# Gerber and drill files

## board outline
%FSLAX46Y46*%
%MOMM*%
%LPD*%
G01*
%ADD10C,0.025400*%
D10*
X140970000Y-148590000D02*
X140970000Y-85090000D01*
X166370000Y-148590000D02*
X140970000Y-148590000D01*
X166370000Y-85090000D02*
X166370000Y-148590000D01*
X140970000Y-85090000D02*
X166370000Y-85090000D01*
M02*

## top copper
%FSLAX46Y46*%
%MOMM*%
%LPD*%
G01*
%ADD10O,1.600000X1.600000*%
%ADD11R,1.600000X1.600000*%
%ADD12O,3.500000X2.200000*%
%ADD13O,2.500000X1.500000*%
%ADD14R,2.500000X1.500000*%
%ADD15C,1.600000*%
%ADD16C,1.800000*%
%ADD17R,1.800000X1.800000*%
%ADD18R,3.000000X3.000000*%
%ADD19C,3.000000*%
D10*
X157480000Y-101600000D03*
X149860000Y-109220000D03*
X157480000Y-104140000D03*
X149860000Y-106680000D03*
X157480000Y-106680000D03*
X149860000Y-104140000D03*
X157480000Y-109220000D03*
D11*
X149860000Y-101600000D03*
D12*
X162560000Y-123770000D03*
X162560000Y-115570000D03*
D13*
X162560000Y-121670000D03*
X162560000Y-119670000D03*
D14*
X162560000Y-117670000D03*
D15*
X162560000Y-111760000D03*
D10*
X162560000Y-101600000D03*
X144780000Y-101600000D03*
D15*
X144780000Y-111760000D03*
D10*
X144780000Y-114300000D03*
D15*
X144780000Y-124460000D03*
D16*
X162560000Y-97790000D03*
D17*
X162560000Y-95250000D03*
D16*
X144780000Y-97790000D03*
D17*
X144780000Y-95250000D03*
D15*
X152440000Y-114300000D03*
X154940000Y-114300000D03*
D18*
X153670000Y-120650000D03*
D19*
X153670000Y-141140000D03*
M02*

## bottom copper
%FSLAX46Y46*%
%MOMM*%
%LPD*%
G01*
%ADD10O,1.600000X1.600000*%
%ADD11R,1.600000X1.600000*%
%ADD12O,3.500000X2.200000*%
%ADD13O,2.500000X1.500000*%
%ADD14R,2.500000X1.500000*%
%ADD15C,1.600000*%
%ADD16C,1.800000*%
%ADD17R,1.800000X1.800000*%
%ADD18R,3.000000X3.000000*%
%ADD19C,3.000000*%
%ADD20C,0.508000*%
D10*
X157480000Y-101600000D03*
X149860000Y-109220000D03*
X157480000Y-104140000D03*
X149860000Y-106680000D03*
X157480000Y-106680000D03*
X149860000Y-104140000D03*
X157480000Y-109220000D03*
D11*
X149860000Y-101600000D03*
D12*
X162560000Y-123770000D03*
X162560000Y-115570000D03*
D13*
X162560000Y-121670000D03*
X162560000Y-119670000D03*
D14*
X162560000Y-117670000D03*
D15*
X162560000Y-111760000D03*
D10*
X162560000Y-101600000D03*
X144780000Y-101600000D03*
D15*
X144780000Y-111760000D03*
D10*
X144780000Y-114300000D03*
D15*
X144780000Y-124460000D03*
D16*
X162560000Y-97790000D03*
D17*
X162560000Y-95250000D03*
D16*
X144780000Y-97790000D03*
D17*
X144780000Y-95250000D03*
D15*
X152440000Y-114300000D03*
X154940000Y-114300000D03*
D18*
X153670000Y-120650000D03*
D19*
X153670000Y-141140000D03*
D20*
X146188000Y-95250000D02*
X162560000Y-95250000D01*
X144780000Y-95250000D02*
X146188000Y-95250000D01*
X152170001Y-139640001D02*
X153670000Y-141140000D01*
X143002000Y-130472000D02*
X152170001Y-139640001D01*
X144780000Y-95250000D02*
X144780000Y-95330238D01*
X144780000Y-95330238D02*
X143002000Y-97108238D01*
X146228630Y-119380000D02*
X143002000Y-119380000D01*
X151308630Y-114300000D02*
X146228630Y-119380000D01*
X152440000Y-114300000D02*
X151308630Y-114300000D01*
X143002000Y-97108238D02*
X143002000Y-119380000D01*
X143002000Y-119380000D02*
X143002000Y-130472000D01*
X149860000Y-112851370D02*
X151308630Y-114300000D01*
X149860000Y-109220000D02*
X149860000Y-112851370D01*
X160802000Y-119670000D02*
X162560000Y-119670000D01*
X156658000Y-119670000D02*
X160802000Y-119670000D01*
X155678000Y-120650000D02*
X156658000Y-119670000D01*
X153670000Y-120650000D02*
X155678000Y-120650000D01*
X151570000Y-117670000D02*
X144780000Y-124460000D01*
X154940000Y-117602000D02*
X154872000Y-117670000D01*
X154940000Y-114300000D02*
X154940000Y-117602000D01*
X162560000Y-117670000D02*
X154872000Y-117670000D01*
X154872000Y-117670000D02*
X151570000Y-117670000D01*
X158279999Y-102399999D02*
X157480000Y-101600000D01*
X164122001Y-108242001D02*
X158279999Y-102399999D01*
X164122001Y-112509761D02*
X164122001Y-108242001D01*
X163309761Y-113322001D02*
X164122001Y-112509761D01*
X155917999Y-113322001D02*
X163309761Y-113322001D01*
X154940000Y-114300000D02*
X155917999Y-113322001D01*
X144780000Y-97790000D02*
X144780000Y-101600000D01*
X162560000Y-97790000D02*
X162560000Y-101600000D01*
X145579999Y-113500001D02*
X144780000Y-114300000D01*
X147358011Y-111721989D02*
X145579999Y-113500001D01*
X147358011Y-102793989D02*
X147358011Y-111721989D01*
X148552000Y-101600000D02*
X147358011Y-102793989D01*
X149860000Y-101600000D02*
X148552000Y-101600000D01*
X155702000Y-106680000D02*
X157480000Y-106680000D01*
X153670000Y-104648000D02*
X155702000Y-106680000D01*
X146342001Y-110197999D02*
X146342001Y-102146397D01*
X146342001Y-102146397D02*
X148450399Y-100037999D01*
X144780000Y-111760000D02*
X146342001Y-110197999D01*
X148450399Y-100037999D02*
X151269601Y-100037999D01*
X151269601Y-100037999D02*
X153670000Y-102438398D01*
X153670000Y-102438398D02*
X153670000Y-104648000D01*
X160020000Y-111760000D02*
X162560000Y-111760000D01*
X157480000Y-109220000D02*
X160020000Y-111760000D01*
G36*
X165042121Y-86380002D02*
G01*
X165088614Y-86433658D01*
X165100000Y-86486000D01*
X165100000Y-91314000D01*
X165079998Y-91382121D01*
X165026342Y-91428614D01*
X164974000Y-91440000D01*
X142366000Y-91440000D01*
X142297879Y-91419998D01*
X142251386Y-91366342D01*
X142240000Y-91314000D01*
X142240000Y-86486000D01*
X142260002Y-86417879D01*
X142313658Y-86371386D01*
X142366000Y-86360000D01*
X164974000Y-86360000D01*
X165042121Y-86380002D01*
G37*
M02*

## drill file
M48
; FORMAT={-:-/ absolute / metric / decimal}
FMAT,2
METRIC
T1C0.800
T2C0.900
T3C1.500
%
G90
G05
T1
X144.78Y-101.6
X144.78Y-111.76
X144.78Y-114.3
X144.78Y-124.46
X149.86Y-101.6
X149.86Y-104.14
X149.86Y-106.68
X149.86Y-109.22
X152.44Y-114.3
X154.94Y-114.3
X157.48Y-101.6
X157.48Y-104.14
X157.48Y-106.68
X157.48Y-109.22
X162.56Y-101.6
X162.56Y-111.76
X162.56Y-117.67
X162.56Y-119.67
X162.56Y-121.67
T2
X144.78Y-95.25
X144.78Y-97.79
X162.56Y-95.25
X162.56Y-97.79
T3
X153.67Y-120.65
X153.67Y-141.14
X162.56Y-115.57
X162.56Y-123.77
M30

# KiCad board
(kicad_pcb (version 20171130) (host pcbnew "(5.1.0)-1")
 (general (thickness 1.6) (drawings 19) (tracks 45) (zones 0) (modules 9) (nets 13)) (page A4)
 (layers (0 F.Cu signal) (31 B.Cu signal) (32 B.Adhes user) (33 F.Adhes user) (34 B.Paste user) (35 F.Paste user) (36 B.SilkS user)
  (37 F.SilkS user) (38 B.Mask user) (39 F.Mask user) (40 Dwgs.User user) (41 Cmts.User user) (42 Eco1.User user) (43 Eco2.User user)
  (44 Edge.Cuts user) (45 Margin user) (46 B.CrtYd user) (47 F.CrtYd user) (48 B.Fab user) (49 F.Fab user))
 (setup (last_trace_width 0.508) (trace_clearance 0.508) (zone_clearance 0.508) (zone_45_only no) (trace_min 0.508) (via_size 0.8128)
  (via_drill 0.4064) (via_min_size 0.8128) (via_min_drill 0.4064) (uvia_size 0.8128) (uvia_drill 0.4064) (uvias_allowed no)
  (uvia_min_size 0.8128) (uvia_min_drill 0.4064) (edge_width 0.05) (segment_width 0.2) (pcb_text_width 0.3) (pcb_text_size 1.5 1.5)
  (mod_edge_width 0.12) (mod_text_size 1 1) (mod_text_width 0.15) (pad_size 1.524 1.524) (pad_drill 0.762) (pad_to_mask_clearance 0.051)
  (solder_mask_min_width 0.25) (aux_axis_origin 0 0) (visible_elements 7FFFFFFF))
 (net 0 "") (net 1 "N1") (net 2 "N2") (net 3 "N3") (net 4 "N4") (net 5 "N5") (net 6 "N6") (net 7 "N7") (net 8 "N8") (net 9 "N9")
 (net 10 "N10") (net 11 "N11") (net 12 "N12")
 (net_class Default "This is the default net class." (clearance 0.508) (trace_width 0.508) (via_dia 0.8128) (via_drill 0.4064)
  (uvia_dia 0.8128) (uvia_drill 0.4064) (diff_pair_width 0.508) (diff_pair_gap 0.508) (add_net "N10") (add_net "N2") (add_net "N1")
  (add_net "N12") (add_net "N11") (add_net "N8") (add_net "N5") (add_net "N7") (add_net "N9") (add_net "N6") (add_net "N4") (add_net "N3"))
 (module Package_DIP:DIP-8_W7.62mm (layer F.Cu) (at 149.86 101.6)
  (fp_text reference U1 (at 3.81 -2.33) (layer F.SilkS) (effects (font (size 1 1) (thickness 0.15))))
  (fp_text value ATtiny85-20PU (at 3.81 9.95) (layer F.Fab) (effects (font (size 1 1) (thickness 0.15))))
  (pad 8 thru_hole oval (at 7.62 0) (size 1.6 1.6) (drill 0.8) (layers *.Cu *.Mask) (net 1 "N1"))
  (pad 4 thru_hole oval (at 0 7.62) (size 1.6 1.6) (drill 0.8) (layers *.Cu *.Mask) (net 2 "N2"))
  (pad 7 thru_hole oval (at 7.62 2.54) (size 1.6 1.6) (drill 0.8) (layers *.Cu *.Mask) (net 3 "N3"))
  (pad 3 thru_hole oval (at 0 5.08) (size 1.6 1.6) (drill 0.8) (layers *.Cu *.Mask) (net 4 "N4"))
  (pad 6 thru_hole oval (at 7.62 5.08) (size 1.6 1.6) (drill 0.8) (layers *.Cu *.Mask) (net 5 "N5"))
  (pad 2 thru_hole oval (at 0 2.54) (size 1.6 1.6) (drill 0.8) (layers *.Cu *.Mask) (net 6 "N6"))
  (pad 5 thru_hole oval (at 7.62 7.62) (size 1.6 1.6) (drill 0.8) (layers *.Cu *.Mask) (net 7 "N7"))
  (pad 1 thru_hole rect (at 0 0) (size 1.6 1.6) (drill 0.8) (layers *.Cu *.Mask) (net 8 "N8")))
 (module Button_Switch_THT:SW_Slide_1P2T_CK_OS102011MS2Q (layer F.Cu) (at 162.56 117.67 270)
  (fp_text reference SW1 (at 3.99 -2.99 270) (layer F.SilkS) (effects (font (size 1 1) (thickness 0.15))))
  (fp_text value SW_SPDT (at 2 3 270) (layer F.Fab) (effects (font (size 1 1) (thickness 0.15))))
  (pad "" thru_hole oval (at 6.1 0 270) (size 2.2 3.5) (drill 1.5) (layers *.Cu *.Mask))
  (pad "" thru_hole oval (at -2.1 0 270) (size 2.2 3.5) (drill 1.5) (layers *.Cu *.Mask))
  (pad 3 thru_hole oval (at 4 0 270) (size 1.5 2.5) (drill 0.8) (layers *.Cu *.Mask) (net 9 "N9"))
  (pad 2 thru_hole oval (at 2 0 270) (size 1.5 2.5) (drill 0.8) (layers *.Cu *.Mask) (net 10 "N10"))
  (pad 1 thru_hole rect (at 0 0 270) (size 1.5 2.5) (drill 0.8) (layers *.Cu *.Mask) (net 1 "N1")))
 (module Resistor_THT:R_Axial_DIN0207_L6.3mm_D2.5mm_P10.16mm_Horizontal (layer F.Cu) (at 162.56 111.76 90)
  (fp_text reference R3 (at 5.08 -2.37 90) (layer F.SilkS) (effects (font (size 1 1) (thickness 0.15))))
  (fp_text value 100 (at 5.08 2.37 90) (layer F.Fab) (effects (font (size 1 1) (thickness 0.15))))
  (pad 1 thru_hole circle (at 0 0 90) (size 1.6 1.6) (drill 0.8) (layers *.Cu *.Mask) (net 7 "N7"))
  (pad 2 thru_hole oval (at 10.16 0 90) (size 1.6 1.6) (drill 0.8) (layers *.Cu *.Mask) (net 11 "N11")))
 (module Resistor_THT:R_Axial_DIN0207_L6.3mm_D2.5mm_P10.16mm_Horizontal (layer F.Cu) (at 144.78 111.76 90)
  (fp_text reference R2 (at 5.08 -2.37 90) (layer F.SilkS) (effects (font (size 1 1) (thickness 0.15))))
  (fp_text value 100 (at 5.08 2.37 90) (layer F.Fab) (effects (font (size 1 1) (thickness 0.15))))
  (pad 2 thru_hole oval (at 10.16 0 90) (size 1.6 1.6) (drill 0.8) (layers *.Cu *.Mask) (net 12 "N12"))
  (pad 1 thru_hole circle (at 0 0 90) (size 1.6 1.6) (drill 0.8) (layers *.Cu *.Mask) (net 5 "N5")))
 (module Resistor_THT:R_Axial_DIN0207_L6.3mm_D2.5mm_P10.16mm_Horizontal (layer F.Cu) (at 144.78 124.46 90)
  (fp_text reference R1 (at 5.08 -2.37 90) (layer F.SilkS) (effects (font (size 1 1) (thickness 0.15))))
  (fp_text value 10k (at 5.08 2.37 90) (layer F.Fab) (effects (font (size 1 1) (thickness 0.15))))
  (pad 2 thru_hole oval (at 10.16 0 90) (size 1.6 1.6) (drill 0.8) (layers *.Cu *.Mask) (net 8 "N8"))
  (pad 1 thru_hole circle (at 0 0 90) (size 1.6 1.6) (drill 0.8) (layers *.Cu *.Mask) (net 1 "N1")))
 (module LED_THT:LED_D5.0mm (layer F.Cu) (at 162.56 95.25 270)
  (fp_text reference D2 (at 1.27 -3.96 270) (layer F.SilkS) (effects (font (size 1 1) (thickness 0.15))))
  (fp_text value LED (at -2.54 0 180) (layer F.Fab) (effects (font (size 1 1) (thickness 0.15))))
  (pad 2 thru_hole circle (at 2.54 0 270) (size 1.8 1.8) (drill 0.9) (layers *.Cu *.Mask) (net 11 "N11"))
  (pad 1 thru_hole rect (at 0 0 270) (size 1.8 1.8) (drill 0.9) (layers *.Cu *.Mask) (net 2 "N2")))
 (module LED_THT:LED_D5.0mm (layer F.Cu) (at 144.78 95.25 270)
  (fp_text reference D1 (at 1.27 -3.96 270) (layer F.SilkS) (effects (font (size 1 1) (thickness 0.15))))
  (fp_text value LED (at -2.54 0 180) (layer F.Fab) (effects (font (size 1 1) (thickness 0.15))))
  (pad 2 thru_hole circle (at 2.54 0 270) (size 1.8 1.8) (drill 0.9) (layers *.Cu *.Mask) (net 12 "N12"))
  (pad 1 thru_hole rect (at 0 0 270) (size 1.8 1.8) (drill 0.9) (layers *.Cu *.Mask) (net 2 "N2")))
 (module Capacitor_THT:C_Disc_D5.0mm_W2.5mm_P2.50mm (layer F.Cu) (at 154.94 114.3 180)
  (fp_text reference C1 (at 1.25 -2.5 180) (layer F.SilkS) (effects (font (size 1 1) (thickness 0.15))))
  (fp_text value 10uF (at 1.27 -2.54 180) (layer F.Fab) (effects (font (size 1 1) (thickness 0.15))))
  (pad 2 thru_hole circle (at 2.5 0 180) (size 1.6 1.6) (drill 0.8) (layers *.Cu *.Mask) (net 2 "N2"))
  (pad 1 thru_hole circle (at 0 0 180) (size 1.6 1.6) (drill 0.8) (layers *.Cu *.Mask) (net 1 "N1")))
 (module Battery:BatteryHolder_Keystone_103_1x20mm (layer F.Cu) (at 153.67 120.65 270)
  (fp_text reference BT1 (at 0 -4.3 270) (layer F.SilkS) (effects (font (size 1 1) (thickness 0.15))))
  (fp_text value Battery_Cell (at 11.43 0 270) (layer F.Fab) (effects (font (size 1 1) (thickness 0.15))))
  (pad 1 thru_hole rect (at 0 0 270) (size 3 3) (drill 1.5) (layers *.Cu *.Mask) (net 10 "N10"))
  (pad 2 thru_hole circle (at 20.49 0 270) (size 3 3) (drill 1.5) (layers *.Cu *.Mask) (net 2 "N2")))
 (gr_line (start 140.97 148.59) (end 140.97 85.09) (layer Edge.Cuts) (width 0.0254))
 (gr_line (start 166.37 148.59) (end 140.97 148.59) (layer Edge.Cuts) (width 0.0254))
 (gr_line (start 166.37 85.09) (end 166.37 148.59) (layer Edge.Cuts) (width 0.0254))
 (gr_line (start 140.97 85.09) (end 166.37 85.09) (layer Edge.Cuts) (width 0.0254))
 (segment (start 146.188 95.25) (end 162.56 95.25) (width 0.508) (layer B.Cu) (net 2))
 (segment (start 144.78 95.25) (end 146.188 95.25) (width 0.508) (layer B.Cu) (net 2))
 (segment (start 152.170001 139.640001) (end 153.67 141.14) (width 0.508) (layer B.Cu) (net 2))
 (segment (start 143.002 130.472) (end 152.170001 139.640001) (width 0.508) (layer B.Cu) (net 2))
 (segment (start 144.78 95.25) (end 144.78 95.330238) (width 0.508) (layer B.Cu) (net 2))
 (segment (start 144.78 95.330238) (end 143.002 97.108238) (width 0.508) (layer B.Cu) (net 2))
 (segment (start 146.22863 119.38) (end 143.002 119.38) (width 0.508) (layer B.Cu) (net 2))
 (segment (start 151.30863 114.3) (end 146.22863 119.38) (width 0.508) (layer B.Cu) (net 2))
 (segment (start 152.44 114.3) (end 151.30863 114.3) (width 0.508) (layer B.Cu) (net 2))
 (segment (start 143.002 97.108238) (end 143.002 119.38) (width 0.508) (layer B.Cu) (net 2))
 (segment (start 143.002 119.38) (end 143.002 130.472) (width 0.508) (layer B.Cu) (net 2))
 (segment (start 149.86 112.85137) (end 151.30863 114.3) (width 0.508) (layer B.Cu) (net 2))
 (segment (start 149.86 109.22) (end 149.86 112.85137) (width 0.508) (layer B.Cu) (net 2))
 (segment (start 160.802 119.67) (end 162.56 119.67) (width 0.508) (layer B.Cu) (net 10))
 (segment (start 156.658 119.67) (end 160.802 119.67) (width 0.508) (layer B.Cu) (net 10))
 (segment (start 155.678 120.65) (end 156.658 119.67) (width 0.508) (layer B.Cu) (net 10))
 (segment (start 153.67 120.65) (end 155.678 120.65) (width 0.508) (layer B.Cu) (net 10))
 (segment (start 151.57 117.67) (end 144.78 124.46) (width 0.508) (layer B.Cu) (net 1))
 (segment (start 154.94 117.602) (end 154.872 117.67) (width 0.508) (layer B.Cu) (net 1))
 (segment (start 154.94 114.3) (end 154.94 117.602) (width 0.508) (layer B.Cu) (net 1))
 (segment (start 162.56 117.67) (end 154.872 117.67) (width 0.508) (layer B.Cu) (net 1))
 (segment (start 154.872 117.67) (end 151.57 117.67) (width 0.508) (layer B.Cu) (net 1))
 (segment (start 158.279999 102.399999) (end 157.48 101.6) (width 0.508) (layer B.Cu) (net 1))
 (segment (start 164.122001 108.242001) (end 158.279999 102.399999) (width 0.508) (layer B.Cu) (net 1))
 (segment (start 164.122001 112.509761) (end 164.122001 108.242001) (width 0.508) (layer B.Cu) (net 1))
 (segment (start 163.309761 113.322001) (end 164.122001 112.509761) (width 0.508) (layer B.Cu) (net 1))
 (segment (start 155.917999 113.322001) (end 163.309761 113.322001) (width 0.508) (layer B.Cu) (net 1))
 (segment (start 154.94 114.3) (end 155.917999 113.322001) (width 0.508) (layer B.Cu) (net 1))
 (segment (start 144.78 97.79) (end 144.78 101.6) (width 0.508) (layer B.Cu) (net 12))
 (segment (start 162.56 97.79) (end 162.56 101.6) (width 0.508) (layer B.Cu) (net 11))
 (segment (start 145.579999 113.500001) (end 144.78 114.3) (width 0.508) (layer B.Cu) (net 8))
 (segment (start 147.358011 111.721989) (end 145.579999 113.500001) (width 0.508) (layer B.Cu) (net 8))
 (segment (start 147.358011 102.793989) (end 147.358011 111.721989) (width 0.508) (layer B.Cu) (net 8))
 (segment (start 148.552 101.6) (end 147.358011 102.793989) (width 0.508) (layer B.Cu) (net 8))
 (segment (start 149.86 101.6) (end 148.552 101.6) (width 0.508) (layer B.Cu) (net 8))
 (segment (start 155.702 106.68) (end 157.48 106.68) (width 0.508) (layer B.Cu) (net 5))
 (segment (start 153.67 104.648) (end 155.702 106.68) (width 0.508) (layer B.Cu) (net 5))
 (segment (start 146.342001 110.197999) (end 146.342001 102.146397) (width 0.508) (layer B.Cu) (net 5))
 (segment (start 146.342001 102.146397) (end 148.450399 100.037999) (width 0.508) (layer B.Cu) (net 5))
 (segment (start 144.78 111.76) (end 146.342001 110.197999) (width 0.508) (layer B.Cu) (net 5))
 (segment (start 148.450399 100.037999) (end 151.269601 100.037999) (width 0.508) (layer B.Cu) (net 5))
 (segment (start 151.269601 100.037999) (end 153.67 102.438398) (width 0.508) (layer B.Cu) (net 5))
 (segment (start 153.67 102.438398) (end 153.67 104.648) (width 0.508) (layer B.Cu) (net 5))
 (segment (start 160.02 111.76) (end 162.56 111.76) (width 0.508) (layer B.Cu) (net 7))
 (segment (start 157.48 109.22) (end 160.02 111.76) (width 0.508) (layer B.Cu) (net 7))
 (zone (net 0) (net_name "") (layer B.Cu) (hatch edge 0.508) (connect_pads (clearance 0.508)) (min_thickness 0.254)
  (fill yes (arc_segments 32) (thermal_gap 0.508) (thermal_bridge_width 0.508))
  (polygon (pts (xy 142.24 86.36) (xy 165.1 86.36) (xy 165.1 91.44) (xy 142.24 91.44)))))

